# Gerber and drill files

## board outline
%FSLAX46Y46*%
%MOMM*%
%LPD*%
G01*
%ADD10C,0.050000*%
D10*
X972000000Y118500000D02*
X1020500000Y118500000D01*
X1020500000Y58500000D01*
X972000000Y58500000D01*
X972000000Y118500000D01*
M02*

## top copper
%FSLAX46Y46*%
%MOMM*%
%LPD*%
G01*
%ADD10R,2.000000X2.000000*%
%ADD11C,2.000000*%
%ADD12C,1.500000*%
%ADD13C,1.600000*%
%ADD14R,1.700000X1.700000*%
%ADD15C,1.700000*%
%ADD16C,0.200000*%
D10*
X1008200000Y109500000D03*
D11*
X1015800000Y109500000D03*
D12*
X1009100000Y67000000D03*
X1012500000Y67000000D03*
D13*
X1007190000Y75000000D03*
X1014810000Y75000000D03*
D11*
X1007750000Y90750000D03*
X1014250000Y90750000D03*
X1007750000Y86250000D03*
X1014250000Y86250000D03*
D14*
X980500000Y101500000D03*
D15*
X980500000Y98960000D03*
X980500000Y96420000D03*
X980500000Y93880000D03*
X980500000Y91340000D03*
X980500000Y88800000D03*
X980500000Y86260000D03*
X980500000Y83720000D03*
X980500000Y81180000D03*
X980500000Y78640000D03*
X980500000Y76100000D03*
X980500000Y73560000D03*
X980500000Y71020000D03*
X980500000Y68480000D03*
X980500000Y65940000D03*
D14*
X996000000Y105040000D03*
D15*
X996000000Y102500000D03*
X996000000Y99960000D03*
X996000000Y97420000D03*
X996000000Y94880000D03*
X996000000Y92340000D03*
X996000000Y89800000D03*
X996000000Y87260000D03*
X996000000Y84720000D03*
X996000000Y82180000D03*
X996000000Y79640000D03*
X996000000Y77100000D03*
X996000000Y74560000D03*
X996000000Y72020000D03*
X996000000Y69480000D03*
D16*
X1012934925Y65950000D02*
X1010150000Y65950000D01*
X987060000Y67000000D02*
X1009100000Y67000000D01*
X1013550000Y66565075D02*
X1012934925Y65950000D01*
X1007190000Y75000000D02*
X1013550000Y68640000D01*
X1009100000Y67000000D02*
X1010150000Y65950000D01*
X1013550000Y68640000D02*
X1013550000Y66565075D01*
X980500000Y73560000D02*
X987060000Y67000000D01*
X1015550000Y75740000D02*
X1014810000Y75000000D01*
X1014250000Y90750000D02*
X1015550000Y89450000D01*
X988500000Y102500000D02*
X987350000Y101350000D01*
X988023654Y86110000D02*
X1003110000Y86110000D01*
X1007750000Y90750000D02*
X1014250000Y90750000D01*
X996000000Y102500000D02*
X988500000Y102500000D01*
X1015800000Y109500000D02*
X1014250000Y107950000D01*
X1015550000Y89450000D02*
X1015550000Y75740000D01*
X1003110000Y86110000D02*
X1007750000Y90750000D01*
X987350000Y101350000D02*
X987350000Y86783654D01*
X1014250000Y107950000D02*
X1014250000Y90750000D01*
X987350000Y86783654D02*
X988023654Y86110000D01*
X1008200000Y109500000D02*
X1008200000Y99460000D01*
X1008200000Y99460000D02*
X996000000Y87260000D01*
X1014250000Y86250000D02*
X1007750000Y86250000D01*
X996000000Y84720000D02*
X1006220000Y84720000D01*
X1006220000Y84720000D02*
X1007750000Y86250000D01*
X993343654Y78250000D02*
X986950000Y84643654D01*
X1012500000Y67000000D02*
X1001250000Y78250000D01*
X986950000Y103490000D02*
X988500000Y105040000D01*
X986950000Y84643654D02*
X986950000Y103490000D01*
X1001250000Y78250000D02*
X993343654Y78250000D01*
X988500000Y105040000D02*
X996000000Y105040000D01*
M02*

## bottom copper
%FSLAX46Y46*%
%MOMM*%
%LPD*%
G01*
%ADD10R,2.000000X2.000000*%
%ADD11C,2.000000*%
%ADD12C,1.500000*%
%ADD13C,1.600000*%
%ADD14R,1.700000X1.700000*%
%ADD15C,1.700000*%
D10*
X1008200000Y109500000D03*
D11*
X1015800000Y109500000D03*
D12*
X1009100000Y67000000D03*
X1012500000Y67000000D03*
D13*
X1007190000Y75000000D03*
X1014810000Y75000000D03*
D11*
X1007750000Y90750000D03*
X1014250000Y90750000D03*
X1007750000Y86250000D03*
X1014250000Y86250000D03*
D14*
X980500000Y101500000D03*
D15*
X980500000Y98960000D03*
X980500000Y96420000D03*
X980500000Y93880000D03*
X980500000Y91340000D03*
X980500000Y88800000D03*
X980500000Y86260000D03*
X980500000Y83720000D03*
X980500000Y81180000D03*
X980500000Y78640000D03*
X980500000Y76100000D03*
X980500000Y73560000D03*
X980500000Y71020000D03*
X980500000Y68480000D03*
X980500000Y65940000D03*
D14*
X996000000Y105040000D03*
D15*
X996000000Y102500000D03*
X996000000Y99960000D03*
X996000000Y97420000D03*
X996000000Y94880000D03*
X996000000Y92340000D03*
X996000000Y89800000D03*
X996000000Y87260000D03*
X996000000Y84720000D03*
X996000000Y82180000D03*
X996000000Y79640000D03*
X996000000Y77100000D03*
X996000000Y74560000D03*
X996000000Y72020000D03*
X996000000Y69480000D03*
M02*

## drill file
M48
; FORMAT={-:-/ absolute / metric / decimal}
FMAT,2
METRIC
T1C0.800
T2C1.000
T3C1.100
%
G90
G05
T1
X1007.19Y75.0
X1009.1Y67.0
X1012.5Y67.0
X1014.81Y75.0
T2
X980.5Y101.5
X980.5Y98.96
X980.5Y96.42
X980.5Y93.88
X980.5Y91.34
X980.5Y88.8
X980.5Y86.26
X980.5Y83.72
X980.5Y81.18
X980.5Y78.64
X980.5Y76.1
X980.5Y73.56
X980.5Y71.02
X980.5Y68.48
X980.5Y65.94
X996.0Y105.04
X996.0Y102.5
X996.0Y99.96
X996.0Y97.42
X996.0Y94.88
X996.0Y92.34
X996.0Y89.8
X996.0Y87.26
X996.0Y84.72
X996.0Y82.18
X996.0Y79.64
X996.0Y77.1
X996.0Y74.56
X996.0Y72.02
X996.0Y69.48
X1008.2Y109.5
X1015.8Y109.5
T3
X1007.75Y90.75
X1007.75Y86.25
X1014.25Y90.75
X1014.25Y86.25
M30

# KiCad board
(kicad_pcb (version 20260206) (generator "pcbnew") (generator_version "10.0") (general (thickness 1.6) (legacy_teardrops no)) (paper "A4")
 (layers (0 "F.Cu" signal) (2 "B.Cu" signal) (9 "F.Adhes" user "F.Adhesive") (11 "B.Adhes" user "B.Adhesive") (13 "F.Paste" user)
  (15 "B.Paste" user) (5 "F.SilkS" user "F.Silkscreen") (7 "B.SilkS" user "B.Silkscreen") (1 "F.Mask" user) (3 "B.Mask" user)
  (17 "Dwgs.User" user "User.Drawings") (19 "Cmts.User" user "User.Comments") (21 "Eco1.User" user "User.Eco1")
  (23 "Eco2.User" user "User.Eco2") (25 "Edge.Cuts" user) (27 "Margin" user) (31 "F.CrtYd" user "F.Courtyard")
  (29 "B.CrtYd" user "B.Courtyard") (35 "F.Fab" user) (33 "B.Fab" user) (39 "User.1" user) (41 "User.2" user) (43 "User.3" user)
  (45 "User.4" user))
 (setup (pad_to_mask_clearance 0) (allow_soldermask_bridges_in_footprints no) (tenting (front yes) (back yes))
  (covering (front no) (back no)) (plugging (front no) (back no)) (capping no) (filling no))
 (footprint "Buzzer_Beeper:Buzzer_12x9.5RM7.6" (layer "F.Cu") (at 1008.2 -109.5)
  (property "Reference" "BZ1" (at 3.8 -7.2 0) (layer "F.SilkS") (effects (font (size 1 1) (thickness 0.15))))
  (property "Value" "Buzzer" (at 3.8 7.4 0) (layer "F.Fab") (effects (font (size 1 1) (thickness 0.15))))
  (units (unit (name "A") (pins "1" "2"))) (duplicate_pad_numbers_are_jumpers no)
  (pad "1" thru_hole rect (at 0 0) (size 2 2) (drill 1) (layers "*.Cu" "*.Mask") (remove_unused_layers no) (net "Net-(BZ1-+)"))
  (pad "2" thru_hole circle (at 7.6 0) (size 2 2) (drill 1) (layers "*.Cu" "*.Mask") (remove_unused_layers no) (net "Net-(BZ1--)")))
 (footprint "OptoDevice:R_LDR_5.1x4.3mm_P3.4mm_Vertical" (layer "F.Cu") (at 1009.1 -67)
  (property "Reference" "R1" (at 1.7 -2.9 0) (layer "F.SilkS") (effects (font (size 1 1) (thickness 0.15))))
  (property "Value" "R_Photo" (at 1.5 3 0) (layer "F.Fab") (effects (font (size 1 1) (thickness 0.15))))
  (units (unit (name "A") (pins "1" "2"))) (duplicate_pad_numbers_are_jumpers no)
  (pad "1" thru_hole circle (at 0 0) (size 1.5 1.5) (drill 0.8) (layers "*.Cu" "*.Mask") (remove_unused_layers no)
   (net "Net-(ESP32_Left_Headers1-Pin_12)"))
  (pad "2" thru_hole circle (at 3.4 0) (size 1.5 1.5) (drill 0.8) (layers "*.Cu" "*.Mask") (remove_unused_layers no)
   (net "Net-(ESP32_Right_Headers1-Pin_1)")))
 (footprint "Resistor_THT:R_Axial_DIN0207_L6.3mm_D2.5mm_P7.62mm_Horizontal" (layer "F.Cu") (at 1007.19 -75)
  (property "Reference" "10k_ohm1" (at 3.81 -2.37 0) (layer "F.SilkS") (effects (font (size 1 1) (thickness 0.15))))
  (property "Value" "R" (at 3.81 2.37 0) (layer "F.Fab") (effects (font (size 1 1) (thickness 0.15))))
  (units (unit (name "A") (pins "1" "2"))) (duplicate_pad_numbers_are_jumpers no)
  (pad "1" thru_hole circle (at 0 0) (size 1.6 1.6) (drill 0.8) (layers "*.Cu" "*.Mask") (remove_unused_layers no)
   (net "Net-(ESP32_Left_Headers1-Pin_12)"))
  (pad "2" thru_hole circle (at 7.62 0) (size 1.6 1.6) (drill 0.8) (layers "*.Cu" "*.Mask") (remove_unused_layers no) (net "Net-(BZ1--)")))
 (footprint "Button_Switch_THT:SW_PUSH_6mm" (layer "F.Cu") (at 1007.75 -90.75)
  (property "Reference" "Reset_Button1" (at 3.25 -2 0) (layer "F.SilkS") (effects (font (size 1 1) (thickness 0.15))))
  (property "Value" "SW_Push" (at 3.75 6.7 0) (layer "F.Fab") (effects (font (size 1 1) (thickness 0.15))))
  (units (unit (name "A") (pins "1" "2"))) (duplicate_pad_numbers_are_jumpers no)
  (pad "1" thru_hole circle (at 0 0 90) (size 2 2) (drill 1.1) (layers "*.Cu" "*.Mask") (remove_unused_layers no) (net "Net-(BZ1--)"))
  (pad "1" thru_hole circle (at 6.5 0 90) (size 2 2) (drill 1.1) (layers "*.Cu" "*.Mask") (remove_unused_layers no) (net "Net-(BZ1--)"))
  (pad "2" thru_hole circle (at 0 4.5 90) (size 2 2) (drill 1.1) (layers "*.Cu" "*.Mask") (remove_unused_layers no)
   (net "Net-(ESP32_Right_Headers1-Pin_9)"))
  (pad "2" thru_hole circle (at 6.5 4.5 90) (size 2 2) (drill 1.1) (layers "*.Cu" "*.Mask") (remove_unused_layers no)
   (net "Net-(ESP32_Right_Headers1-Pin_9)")))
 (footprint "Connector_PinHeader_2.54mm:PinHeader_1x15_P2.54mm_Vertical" (layer "F.Cu") (at 980.5 -101.5)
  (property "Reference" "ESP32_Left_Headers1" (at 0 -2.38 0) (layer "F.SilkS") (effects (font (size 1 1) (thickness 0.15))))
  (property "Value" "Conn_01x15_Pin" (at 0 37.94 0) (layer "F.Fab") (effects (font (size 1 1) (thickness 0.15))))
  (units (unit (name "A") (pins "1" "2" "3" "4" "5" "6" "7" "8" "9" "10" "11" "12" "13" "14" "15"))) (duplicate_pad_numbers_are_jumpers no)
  (pad "1" thru_hole rect (at 0 0) (size 1.7 1.7) (drill 1) (layers "*.Cu" "*.Mask") (remove_unused_layers no)
   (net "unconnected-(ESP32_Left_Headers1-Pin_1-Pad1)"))
  (pad "2" thru_hole circle (at 0 2.54) (size 1.7 1.7) (drill 1) (layers "*.Cu" "*.Mask") (remove_unused_layers no)
   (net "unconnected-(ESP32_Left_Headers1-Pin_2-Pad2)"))
  (pad "3" thru_hole circle (at 0 5.08) (size 1.7 1.7) (drill 1) (layers "*.Cu" "*.Mask") (remove_unused_layers no)
   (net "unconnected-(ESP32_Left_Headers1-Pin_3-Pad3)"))
  (pad "4" thru_hole circle (at 0 7.62) (size 1.7 1.7) (drill 1) (layers "*.Cu" "*.Mask") (remove_unused_layers no)
   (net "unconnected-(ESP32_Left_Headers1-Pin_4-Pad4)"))
  (pad "5" thru_hole circle (at 0 10.16) (size 1.7 1.7) (drill 1) (layers "*.Cu" "*.Mask") (remove_unused_layers no)
   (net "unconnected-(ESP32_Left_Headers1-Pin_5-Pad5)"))
  (pad "6" thru_hole circle (at 0 12.7) (size 1.7 1.7) (drill 1) (layers "*.Cu" "*.Mask") (remove_unused_layers no)
   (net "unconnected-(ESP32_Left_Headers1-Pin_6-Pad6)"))
  (pad "7" thru_hole circle (at 0 15.24) (size 1.7 1.7) (drill 1) (layers "*.Cu" "*.Mask") (remove_unused_layers no)
   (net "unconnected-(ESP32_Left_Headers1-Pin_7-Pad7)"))
  (pad "8" thru_hole circle (at 0 17.78) (size 1.7 1.7) (drill 1) (layers "*.Cu" "*.Mask") (remove_unused_layers no)
   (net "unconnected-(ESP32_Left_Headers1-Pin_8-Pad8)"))
  (pad "9" thru_hole circle (at 0 20.32) (size 1.7 1.7) (drill 1) (layers "*.Cu" "*.Mask") (remove_unused_layers no)
   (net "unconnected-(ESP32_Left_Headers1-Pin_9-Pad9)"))
  (pad "10" thru_hole circle (at 0 22.86) (size 1.7 1.7) (drill 1) (layers "*.Cu" "*.Mask") (remove_unused_layers no)
   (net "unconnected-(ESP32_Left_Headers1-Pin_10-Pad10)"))
  (pad "11" thru_hole circle (at 0 25.4) (size 1.7 1.7) (drill 1) (layers "*.Cu" "*.Mask") (remove_unused_layers no)
   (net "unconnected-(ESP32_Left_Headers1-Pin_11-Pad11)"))
  (pad "12" thru_hole circle (at 0 27.94) (size 1.7 1.7) (drill 1) (layers "*.Cu" "*.Mask") (remove_unused_layers no)
   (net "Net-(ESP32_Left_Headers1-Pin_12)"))
  (pad "13" thru_hole circle (at 0 30.48) (size 1.7 1.7) (drill 1) (layers "*.Cu" "*.Mask") (remove_unused_layers no)
   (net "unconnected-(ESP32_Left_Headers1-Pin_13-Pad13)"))
  (pad "14" thru_hole circle (at 0 33.02) (size 1.7 1.7) (drill 1) (layers "*.Cu" "*.Mask") (remove_unused_layers no)
   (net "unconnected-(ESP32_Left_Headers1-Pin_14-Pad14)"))
  (pad "15" thru_hole circle (at 0 35.56) (size 1.7 1.7) (drill 1) (layers "*.Cu" "*.Mask") (remove_unused_layers no)
   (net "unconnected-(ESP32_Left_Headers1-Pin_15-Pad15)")))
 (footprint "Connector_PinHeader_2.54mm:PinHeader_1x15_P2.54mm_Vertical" (layer "F.Cu") (at 996 -105.04)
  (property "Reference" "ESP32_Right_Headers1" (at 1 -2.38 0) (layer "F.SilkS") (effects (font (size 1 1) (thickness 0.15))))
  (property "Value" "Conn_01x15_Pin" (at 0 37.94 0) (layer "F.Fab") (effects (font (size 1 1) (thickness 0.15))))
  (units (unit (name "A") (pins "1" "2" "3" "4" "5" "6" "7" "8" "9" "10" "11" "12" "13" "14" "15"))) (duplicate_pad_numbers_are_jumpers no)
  (pad "1" thru_hole rect (at 0 0) (size 1.7 1.7) (drill 1) (layers "*.Cu" "*.Mask") (remove_unused_layers no)
   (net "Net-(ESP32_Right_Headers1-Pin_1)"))
  (pad "2" thru_hole circle (at 0 2.54) (size 1.7 1.7) (drill 1) (layers "*.Cu" "*.Mask") (remove_unused_layers no) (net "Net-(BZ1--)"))
  (pad "3" thru_hole circle (at 0 5.08) (size 1.7 1.7) (drill 1) (layers "*.Cu" "*.Mask") (remove_unused_layers no)
   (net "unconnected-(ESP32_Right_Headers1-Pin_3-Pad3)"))
  (pad "4" thru_hole circle (at 0 7.62) (size 1.7 1.7) (drill 1) (layers "*.Cu" "*.Mask") (remove_unused_layers no)
   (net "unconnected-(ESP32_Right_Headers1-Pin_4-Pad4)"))
  (pad "5" thru_hole circle (at 0 10.16) (size 1.7 1.7) (drill 1) (layers "*.Cu" "*.Mask") (remove_unused_layers no)
   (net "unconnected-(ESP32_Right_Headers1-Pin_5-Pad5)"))
  (pad "6" thru_hole circle (at 0 12.7) (size 1.7 1.7) (drill 1) (layers "*.Cu" "*.Mask") (remove_unused_layers no)
   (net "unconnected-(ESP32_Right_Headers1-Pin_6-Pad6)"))
  (pad "7" thru_hole circle (at 0 15.24) (size 1.7 1.7) (drill 1) (layers "*.Cu" "*.Mask") (remove_unused_layers no)
   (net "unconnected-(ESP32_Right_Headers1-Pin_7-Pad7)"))
  (pad "8" thru_hole circle (at 0 17.78) (size 1.7 1.7) (drill 1) (layers "*.Cu" "*.Mask") (remove_unused_layers no) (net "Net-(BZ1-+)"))
  (pad "9" thru_hole circle (at 0 20.32) (size 1.7 1.7) (drill 1) (layers "*.Cu" "*.Mask") (remove_unused_layers no)
   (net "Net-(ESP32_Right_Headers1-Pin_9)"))
  (pad "10" thru_hole circle (at 0 22.86) (size 1.7 1.7) (drill 1) (layers "*.Cu" "*.Mask") (remove_unused_layers no)
   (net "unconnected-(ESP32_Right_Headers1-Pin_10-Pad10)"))
  (pad "11" thru_hole circle (at 0 25.4) (size 1.7 1.7) (drill 1) (layers "*.Cu" "*.Mask") (remove_unused_layers no)
   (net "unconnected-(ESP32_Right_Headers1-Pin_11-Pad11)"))
  (pad "12" thru_hole circle (at 0 27.94) (size 1.7 1.7) (drill 1) (layers "*.Cu" "*.Mask") (remove_unused_layers no)
   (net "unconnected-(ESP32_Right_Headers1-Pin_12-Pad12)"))
  (pad "13" thru_hole circle (at 0 30.48) (size 1.7 1.7) (drill 1) (layers "*.Cu" "*.Mask") (remove_unused_layers no)
   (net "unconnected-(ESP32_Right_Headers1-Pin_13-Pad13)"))
  (pad "14" thru_hole circle (at 0 33.02) (size 1.7 1.7) (drill 1) (layers "*.Cu" "*.Mask") (remove_unused_layers no)
   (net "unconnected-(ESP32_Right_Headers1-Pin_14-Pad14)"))
  (pad "15" thru_hole circle (at 0 35.56) (size 1.7 1.7) (drill 1) (layers "*.Cu" "*.Mask") (remove_unused_layers no)
   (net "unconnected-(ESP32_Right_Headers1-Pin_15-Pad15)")))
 (gr_rect (start 972 -118.5) (end 1020.5 -58.5) (stroke (width 0.05) (type default)) (fill no) (layer "Edge.Cuts"))
 (segment (start 1012.934925 -65.95) (end 1010.15 -65.95) (width 0.2) (layer "F.Cu") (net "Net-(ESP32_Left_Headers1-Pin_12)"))
 (segment (start 987.06 -67) (end 1009.1 -67) (width 0.2) (layer "F.Cu") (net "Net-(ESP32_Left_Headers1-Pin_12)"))
 (segment (start 1013.55 -66.565075) (end 1012.934925 -65.95) (width 0.2) (layer "F.Cu") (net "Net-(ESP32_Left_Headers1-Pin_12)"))
 (segment (start 1007.19 -75) (end 1013.55 -68.64) (width 0.2) (layer "F.Cu") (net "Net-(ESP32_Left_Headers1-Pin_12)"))
 (segment (start 1009.1 -67) (end 1010.15 -65.95) (width 0.2) (layer "F.Cu") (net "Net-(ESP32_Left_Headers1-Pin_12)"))
 (segment (start 1013.55 -68.64) (end 1013.55 -66.565075) (width 0.2) (layer "F.Cu") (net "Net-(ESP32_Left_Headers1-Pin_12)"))
 (segment (start 980.5 -73.56) (end 987.06 -67) (width 0.2) (layer "F.Cu") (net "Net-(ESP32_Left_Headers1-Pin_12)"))
 (segment (start 1015.55 -75.74) (end 1014.81 -75) (width 0.2) (layer "F.Cu") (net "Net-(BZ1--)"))
 (segment (start 1014.25 -90.75) (end 1015.55 -89.45) (width 0.2) (layer "F.Cu") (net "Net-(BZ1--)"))
 (segment (start 988.5 -102.5) (end 987.35 -101.35) (width 0.2) (layer "F.Cu") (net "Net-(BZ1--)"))
 (segment (start 988.023654 -86.11) (end 1003.11 -86.11) (width 0.2) (layer "F.Cu") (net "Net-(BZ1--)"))
 (segment (start 1007.75 -90.75) (end 1014.25 -90.75) (width 0.2) (layer "F.Cu") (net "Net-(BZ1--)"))
 (segment (start 996 -102.5) (end 988.5 -102.5) (width 0.2) (layer "F.Cu") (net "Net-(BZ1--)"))
 (segment (start 1015.8 -109.5) (end 1014.25 -107.95) (width 0.2) (layer "F.Cu") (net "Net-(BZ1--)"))
 (segment (start 1015.55 -89.45) (end 1015.55 -75.74) (width 0.2) (layer "F.Cu") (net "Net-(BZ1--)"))
 (segment (start 1003.11 -86.11) (end 1007.75 -90.75) (width 0.2) (layer "F.Cu") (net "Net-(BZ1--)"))
 (segment (start 987.35 -101.35) (end 987.35 -86.783654) (width 0.2) (layer "F.Cu") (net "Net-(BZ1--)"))
 (segment (start 1014.25 -107.95) (end 1014.25 -90.75) (width 0.2) (layer "F.Cu") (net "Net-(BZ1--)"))
 (segment (start 987.35 -86.783654) (end 988.023654 -86.11) (width 0.2) (layer "F.Cu") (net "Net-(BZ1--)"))
 (segment (start 1008.2 -109.5) (end 1008.2 -99.46) (width 0.2) (layer "F.Cu") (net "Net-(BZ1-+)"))
 (segment (start 1008.2 -99.46) (end 996 -87.26) (width 0.2) (layer "F.Cu") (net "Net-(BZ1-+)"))
 (segment (start 1014.25 -86.25) (end 1007.75 -86.25) (width 0.2) (layer "F.Cu") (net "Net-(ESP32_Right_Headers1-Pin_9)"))
 (segment (start 996 -84.72) (end 1006.22 -84.72) (width 0.2) (layer "F.Cu") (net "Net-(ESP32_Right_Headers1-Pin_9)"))
 (segment (start 1006.22 -84.72) (end 1007.75 -86.25) (width 0.2) (layer "F.Cu") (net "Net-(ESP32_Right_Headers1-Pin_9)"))
 (segment (start 993.343654 -78.25) (end 986.95 -84.643654) (width 0.2) (layer "F.Cu") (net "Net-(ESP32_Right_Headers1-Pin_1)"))
 (segment (start 1012.5 -67) (end 1001.25 -78.25) (width 0.2) (layer "F.Cu") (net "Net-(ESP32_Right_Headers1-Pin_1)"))
 (segment (start 986.95 -103.49) (end 988.5 -105.04) (width 0.2) (layer "F.Cu") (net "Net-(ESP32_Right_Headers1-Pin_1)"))
 (segment (start 986.95 -84.643654) (end 986.95 -103.49) (width 0.2) (layer "F.Cu") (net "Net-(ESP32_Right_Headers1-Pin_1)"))
 (segment (start 1001.25 -78.25) (end 993.343654 -78.25) (width 0.2) (layer "F.Cu") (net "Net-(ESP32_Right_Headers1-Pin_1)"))
 (segment (start 988.5 -105.04) (end 996 -105.04) (width 0.2) (layer "F.Cu") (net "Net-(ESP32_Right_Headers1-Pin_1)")))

